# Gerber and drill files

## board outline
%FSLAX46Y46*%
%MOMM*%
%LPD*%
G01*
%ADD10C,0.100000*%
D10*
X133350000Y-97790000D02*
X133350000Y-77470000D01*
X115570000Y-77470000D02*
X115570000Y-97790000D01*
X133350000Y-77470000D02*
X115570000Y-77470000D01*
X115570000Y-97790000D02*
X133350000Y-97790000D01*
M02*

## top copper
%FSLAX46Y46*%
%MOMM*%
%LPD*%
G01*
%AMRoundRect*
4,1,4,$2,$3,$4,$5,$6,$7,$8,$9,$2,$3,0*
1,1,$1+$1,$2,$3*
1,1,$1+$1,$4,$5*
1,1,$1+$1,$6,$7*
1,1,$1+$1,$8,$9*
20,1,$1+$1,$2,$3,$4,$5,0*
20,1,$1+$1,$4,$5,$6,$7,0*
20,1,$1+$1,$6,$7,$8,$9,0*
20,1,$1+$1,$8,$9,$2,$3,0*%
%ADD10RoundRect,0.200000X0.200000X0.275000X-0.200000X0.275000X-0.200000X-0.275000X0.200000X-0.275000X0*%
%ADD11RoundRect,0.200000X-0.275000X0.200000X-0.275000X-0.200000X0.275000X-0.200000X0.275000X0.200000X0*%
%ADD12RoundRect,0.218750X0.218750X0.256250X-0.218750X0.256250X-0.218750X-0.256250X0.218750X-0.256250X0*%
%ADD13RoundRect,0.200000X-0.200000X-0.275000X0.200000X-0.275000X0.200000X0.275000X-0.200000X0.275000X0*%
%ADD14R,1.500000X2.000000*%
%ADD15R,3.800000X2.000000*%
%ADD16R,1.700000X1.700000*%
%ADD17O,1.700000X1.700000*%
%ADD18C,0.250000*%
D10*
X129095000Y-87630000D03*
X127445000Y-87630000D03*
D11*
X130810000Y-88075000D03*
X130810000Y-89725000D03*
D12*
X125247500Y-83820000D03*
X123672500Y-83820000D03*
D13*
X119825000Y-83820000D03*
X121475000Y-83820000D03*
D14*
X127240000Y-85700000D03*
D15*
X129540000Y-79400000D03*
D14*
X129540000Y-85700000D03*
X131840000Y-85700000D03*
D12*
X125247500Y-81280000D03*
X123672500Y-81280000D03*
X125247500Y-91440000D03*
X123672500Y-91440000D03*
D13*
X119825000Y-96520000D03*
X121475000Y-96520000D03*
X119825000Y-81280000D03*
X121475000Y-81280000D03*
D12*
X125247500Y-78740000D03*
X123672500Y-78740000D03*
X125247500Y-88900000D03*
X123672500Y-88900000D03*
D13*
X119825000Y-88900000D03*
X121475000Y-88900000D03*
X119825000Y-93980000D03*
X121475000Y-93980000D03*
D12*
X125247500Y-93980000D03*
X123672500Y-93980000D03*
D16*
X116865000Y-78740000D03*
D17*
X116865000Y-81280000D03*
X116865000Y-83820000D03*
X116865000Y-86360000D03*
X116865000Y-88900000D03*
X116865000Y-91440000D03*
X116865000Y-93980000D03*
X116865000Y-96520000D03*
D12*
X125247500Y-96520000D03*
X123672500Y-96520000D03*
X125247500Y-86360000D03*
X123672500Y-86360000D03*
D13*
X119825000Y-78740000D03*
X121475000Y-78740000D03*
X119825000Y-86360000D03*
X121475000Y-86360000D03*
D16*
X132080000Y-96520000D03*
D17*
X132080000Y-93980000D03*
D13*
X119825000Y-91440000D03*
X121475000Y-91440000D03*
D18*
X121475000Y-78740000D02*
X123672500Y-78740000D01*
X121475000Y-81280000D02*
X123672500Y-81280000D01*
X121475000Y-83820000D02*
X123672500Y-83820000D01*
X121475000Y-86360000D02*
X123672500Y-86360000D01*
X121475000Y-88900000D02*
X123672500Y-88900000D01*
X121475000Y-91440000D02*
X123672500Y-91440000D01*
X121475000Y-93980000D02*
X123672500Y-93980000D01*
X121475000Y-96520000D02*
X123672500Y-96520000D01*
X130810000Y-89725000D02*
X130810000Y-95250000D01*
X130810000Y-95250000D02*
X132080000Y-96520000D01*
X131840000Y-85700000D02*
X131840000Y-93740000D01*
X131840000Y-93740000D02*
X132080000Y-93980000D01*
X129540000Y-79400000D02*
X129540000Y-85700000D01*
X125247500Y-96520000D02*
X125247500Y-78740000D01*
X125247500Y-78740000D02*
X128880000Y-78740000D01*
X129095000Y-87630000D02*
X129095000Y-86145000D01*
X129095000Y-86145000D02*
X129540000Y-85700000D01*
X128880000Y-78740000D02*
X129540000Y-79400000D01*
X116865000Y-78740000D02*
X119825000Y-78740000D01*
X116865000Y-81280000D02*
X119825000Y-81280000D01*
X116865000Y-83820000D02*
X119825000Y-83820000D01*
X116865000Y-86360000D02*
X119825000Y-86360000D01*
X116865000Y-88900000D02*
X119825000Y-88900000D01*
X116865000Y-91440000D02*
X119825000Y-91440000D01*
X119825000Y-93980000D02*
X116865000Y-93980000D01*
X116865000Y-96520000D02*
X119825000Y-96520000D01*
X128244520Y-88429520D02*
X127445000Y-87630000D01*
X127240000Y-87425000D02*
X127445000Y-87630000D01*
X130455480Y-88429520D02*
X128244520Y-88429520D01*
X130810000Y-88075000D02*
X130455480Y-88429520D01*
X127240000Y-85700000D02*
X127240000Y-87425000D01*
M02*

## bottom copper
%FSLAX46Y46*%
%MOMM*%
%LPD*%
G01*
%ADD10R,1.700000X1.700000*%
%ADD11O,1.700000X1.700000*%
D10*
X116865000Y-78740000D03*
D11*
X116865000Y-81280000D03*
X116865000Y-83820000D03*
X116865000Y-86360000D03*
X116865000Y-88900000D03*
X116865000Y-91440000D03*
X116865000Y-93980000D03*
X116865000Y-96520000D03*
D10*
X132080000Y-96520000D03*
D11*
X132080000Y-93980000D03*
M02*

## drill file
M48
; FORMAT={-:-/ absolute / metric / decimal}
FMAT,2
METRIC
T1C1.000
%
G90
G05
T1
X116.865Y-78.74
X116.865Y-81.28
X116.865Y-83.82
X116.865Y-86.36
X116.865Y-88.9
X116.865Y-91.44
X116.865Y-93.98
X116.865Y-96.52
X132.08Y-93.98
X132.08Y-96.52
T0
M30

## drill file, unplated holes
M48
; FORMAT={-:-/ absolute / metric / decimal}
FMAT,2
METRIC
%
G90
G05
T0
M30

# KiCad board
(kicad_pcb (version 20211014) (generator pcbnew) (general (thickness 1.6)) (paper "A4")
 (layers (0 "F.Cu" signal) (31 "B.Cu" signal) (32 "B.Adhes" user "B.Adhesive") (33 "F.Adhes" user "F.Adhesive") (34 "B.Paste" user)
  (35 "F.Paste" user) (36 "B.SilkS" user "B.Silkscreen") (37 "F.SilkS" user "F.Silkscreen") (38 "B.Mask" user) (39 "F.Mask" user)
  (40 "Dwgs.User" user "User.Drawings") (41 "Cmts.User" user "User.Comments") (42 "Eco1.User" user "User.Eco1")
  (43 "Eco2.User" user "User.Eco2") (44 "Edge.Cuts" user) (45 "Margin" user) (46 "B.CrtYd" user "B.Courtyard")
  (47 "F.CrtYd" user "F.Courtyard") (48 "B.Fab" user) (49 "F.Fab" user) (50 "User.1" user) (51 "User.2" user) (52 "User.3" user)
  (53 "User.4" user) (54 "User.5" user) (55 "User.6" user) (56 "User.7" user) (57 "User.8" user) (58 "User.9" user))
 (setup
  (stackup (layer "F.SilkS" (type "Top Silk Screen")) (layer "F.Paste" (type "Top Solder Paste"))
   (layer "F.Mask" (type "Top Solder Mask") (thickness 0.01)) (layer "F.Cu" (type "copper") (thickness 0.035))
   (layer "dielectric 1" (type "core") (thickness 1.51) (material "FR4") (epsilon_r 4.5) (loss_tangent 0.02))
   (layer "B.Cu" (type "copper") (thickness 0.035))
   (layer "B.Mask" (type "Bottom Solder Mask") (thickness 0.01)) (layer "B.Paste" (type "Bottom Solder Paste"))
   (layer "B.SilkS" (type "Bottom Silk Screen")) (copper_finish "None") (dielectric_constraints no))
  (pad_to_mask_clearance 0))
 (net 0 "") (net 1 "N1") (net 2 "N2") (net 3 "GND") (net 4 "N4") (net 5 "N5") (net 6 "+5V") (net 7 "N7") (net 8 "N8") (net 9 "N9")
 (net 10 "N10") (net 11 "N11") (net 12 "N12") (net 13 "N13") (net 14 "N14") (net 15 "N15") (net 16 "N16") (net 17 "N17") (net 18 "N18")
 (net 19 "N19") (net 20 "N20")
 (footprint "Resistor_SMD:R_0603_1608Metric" (layer "F.Cu") (at 128.27 87.63 180)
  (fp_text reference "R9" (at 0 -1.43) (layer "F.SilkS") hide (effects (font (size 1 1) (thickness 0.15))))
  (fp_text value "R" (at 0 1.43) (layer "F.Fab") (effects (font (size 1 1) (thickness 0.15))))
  (pad "1" smd roundrect locked (at -0.825 0 180) (size 0.8 0.95) (layers "F.Cu" "F.Paste" "F.Mask") (roundrect_rratio 0.25) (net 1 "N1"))
  (pad "2" smd roundrect locked (at 0.825 0 180) (size 0.8 0.95) (layers "F.Cu" "F.Paste" "F.Mask") (roundrect_rratio 0.25) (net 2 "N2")))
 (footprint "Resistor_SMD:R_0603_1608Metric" (layer "F.Cu") (at 130.81 88.9 -90)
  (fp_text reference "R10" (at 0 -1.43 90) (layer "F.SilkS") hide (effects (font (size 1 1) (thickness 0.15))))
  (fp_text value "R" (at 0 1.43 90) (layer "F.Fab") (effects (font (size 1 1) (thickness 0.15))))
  (pad "1" smd roundrect locked (at -0.825 0 270) (size 0.8 0.95) (layers "F.Cu" "F.Paste" "F.Mask") (roundrect_rratio 0.25) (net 2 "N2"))
  (pad "2" smd roundrect locked (at 0.825 0 270) (size 0.8 0.95) (layers "F.Cu" "F.Paste" "F.Mask") (roundrect_rratio 0.25) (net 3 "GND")))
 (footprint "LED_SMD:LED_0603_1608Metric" (layer "F.Cu") (at 124.46 83.82 180)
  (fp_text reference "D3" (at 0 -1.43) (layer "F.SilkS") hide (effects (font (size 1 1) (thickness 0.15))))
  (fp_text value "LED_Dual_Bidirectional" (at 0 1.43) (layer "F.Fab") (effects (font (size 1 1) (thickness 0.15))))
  (pad "1" smd roundrect locked (at -0.7875 0 180) (size 0.875 0.95) (layers "F.Cu" "F.Paste" "F.Mask") (roundrect_rratio 0.25) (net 1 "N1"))
  (pad "2" smd roundrect locked (at 0.7875 0 180) (size 0.875 0.95) (layers "F.Cu" "F.Paste" "F.Mask") (roundrect_rratio 0.25) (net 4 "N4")))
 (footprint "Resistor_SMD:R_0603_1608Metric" (layer "F.Cu") (at 120.65 83.82)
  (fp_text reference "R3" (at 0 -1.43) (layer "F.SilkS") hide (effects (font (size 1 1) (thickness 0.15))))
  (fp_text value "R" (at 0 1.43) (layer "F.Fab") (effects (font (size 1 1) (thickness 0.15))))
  (pad "1" smd roundrect locked (at -0.825 0) (size 0.8 0.95) (layers "F.Cu" "F.Paste" "F.Mask") (roundrect_rratio 0.25) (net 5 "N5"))
  (pad "2" smd roundrect locked (at 0.825 0) (size 0.8 0.95) (layers "F.Cu" "F.Paste" "F.Mask") (roundrect_rratio 0.25) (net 4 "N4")))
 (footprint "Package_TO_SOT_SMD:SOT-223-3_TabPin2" (layer "F.Cu") (at 129.54 82.55 90)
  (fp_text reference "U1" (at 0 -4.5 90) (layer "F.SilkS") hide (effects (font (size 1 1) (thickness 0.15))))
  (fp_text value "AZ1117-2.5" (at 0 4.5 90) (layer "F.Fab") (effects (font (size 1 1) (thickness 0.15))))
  (pad "1" smd rect locked (at -3.15 -2.3 90) (size 2 1.5) (layers "F.Cu" "F.Paste" "F.Mask") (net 2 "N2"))
  (pad "2" smd rect locked (at 3.15 0 90) (size 2 3.8) (layers "F.Cu" "F.Paste" "F.Mask") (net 1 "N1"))
  (pad "2" smd rect locked (at -3.15 0 90) (size 2 1.5) (layers "F.Cu" "F.Paste" "F.Mask") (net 1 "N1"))
  (pad "3" smd rect locked (at -3.15 2.3 90) (size 2 1.5) (layers "F.Cu" "F.Paste" "F.Mask") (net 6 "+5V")))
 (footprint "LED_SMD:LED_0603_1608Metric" (layer "F.Cu") (at 124.46 81.28 180)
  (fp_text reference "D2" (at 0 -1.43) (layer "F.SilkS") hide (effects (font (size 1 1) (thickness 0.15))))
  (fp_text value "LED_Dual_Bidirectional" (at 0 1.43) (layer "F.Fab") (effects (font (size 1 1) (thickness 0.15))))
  (pad "1" smd roundrect locked (at -0.7875 0 180) (size 0.875 0.95) (layers "F.Cu" "F.Paste" "F.Mask") (roundrect_rratio 0.25) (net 1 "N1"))
  (pad "2" smd roundrect locked (at 0.7875 0 180) (size 0.875 0.95) (layers "F.Cu" "F.Paste" "F.Mask") (roundrect_rratio 0.25) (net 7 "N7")))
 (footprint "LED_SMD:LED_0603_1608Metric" (layer "F.Cu") (at 124.46 91.44 180)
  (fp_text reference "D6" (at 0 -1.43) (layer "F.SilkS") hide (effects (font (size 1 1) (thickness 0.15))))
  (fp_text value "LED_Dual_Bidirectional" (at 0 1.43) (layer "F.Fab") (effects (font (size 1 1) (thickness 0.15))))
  (pad "1" smd roundrect locked (at -0.7875 0 180) (size 0.875 0.95) (layers "F.Cu" "F.Paste" "F.Mask") (roundrect_rratio 0.25) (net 1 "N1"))
  (pad "2" smd roundrect locked (at 0.7875 0 180) (size 0.875 0.95) (layers "F.Cu" "F.Paste" "F.Mask") (roundrect_rratio 0.25) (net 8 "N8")))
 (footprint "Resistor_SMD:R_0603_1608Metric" (layer "F.Cu") (at 120.65 96.52)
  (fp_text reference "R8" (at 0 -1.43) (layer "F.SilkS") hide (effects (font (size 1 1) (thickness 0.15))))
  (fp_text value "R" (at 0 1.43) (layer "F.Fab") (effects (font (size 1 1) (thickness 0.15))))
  (pad "1" smd roundrect locked (at -0.825 0) (size 0.8 0.95) (layers "F.Cu" "F.Paste" "F.Mask") (roundrect_rratio 0.25) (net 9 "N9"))
  (pad "2" smd roundrect locked (at 0.825 0) (size 0.8 0.95) (layers "F.Cu" "F.Paste" "F.Mask") (roundrect_rratio 0.25) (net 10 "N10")))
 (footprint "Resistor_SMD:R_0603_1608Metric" (layer "F.Cu") (at 120.65 81.28)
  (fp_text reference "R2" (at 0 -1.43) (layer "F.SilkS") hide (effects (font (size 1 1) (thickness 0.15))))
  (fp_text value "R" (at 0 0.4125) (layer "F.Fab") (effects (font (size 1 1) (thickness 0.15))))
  (pad "1" smd roundrect locked (at -0.825 0) (size 0.8 0.95) (layers "F.Cu" "F.Paste" "F.Mask") (roundrect_rratio 0.25) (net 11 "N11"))
  (pad "2" smd roundrect locked (at 0.825 0) (size 0.8 0.95) (layers "F.Cu" "F.Paste" "F.Mask") (roundrect_rratio 0.25) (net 7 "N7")))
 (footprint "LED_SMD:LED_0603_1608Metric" (layer "F.Cu") (at 124.46 78.74 180)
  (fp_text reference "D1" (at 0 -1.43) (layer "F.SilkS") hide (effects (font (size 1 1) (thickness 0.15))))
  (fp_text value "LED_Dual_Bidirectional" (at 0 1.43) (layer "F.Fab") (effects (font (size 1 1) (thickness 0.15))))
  (pad "1" smd roundrect locked (at -0.7875 0 180) (size 0.875 0.95) (layers "F.Cu" "F.Paste" "F.Mask") (roundrect_rratio 0.25) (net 1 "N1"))
  (pad "2" smd roundrect locked (at 0.7875 0 180) (size 0.875 0.95) (layers "F.Cu" "F.Paste" "F.Mask") (roundrect_rratio 0.25)
   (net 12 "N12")))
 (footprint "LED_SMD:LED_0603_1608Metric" (layer "F.Cu") (at 124.46 88.9 180)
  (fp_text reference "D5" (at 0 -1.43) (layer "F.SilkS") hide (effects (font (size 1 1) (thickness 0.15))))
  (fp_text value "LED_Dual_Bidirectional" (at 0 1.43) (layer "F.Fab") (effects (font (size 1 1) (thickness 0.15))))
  (pad "1" smd roundrect locked (at -0.7875 0 180) (size 0.875 0.95) (layers "F.Cu" "F.Paste" "F.Mask") (roundrect_rratio 0.25) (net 1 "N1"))
  (pad "2" smd roundrect locked (at 0.7875 0 180) (size 0.875 0.95) (layers "F.Cu" "F.Paste" "F.Mask") (roundrect_rratio 0.25)
   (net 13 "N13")))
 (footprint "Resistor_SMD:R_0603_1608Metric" (layer "F.Cu") (at 120.65 88.9)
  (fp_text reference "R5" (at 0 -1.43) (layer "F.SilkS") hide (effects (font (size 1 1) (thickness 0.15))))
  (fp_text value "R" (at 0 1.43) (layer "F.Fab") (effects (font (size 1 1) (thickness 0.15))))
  (pad "1" smd roundrect locked (at -0.825 0) (size 0.8 0.95) (layers "F.Cu" "F.Paste" "F.Mask") (roundrect_rratio 0.25) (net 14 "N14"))
  (pad "2" smd roundrect locked (at 0.825 0) (size 0.8 0.95) (layers "F.Cu" "F.Paste" "F.Mask") (roundrect_rratio 0.25) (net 13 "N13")))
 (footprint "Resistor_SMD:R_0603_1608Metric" (layer "F.Cu") (at 120.65 93.98)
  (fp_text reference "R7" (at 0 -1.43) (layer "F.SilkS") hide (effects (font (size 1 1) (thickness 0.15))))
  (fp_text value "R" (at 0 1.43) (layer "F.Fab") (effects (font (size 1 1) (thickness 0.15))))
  (pad "1" smd roundrect locked (at -0.825 0) (size 0.8 0.95) (layers "F.Cu" "F.Paste" "F.Mask") (roundrect_rratio 0.25) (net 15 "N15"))
  (pad "2" smd roundrect locked (at 0.825 0) (size 0.8 0.95) (layers "F.Cu" "F.Paste" "F.Mask") (roundrect_rratio 0.25) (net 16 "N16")))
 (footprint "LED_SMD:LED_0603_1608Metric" (layer "F.Cu") (at 124.46 93.98 180)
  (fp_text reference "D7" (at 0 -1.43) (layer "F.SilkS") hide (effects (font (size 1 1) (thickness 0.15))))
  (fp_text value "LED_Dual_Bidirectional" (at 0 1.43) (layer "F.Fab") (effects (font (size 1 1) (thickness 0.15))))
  (pad "1" smd roundrect locked (at -0.7875 0 180) (size 0.875 0.95) (layers "F.Cu" "F.Paste" "F.Mask") (roundrect_rratio 0.25) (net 1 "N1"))
  (pad "2" smd roundrect locked (at 0.7875 0 180) (size 0.875 0.95) (layers "F.Cu" "F.Paste" "F.Mask") (roundrect_rratio 0.25)
   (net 16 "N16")))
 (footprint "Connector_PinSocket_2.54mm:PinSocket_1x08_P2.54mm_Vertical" (layer "F.Cu") (at 116.865 78.74)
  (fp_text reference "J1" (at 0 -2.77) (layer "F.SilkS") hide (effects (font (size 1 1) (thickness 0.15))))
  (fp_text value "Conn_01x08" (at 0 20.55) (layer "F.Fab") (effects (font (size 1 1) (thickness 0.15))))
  (pad "1" thru_hole rect locked (at 0 0) (size 1.7 1.7) (drill 1) (layers *.Cu *.Mask) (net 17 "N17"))
  (pad "2" thru_hole oval locked (at 0 2.54) (size 1.7 1.7) (drill 1) (layers *.Cu *.Mask) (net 11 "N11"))
  (pad "3" thru_hole oval locked (at 0 5.08) (size 1.7 1.7) (drill 1) (layers *.Cu *.Mask) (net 5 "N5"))
  (pad "4" thru_hole oval locked (at 0 7.62) (size 1.7 1.7) (drill 1) (layers *.Cu *.Mask) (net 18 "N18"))
  (pad "5" thru_hole oval locked (at 0 10.16) (size 1.7 1.7) (drill 1) (layers *.Cu *.Mask) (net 14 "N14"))
  (pad "6" thru_hole oval locked (at 0 12.7) (size 1.7 1.7) (drill 1) (layers *.Cu *.Mask) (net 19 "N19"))
  (pad "7" thru_hole oval locked (at 0 15.24) (size 1.7 1.7) (drill 1) (layers *.Cu *.Mask) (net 15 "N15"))
  (pad "8" thru_hole oval locked (at 0 17.78) (size 1.7 1.7) (drill 1) (layers *.Cu *.Mask) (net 9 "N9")))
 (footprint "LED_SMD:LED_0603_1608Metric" (layer "F.Cu") (at 124.46 96.52 180)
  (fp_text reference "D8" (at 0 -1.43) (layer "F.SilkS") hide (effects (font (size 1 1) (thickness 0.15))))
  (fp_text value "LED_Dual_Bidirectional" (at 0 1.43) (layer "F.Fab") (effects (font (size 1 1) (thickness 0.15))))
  (pad "1" smd roundrect locked (at -0.7875 0 180) (size 0.875 0.95) (layers "F.Cu" "F.Paste" "F.Mask") (roundrect_rratio 0.25) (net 1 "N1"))
  (pad "2" smd roundrect locked (at 0.7875 0 180) (size 0.875 0.95) (layers "F.Cu" "F.Paste" "F.Mask") (roundrect_rratio 0.25)
   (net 10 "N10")))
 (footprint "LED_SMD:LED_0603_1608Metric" (layer "F.Cu") (at 124.46 86.36 180)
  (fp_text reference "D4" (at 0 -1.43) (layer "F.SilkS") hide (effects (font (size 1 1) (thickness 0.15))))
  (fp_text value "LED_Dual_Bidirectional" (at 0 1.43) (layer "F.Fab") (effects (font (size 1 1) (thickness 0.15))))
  (pad "1" smd roundrect locked (at -0.7875 0 180) (size 0.875 0.95) (layers "F.Cu" "F.Paste" "F.Mask") (roundrect_rratio 0.25) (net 1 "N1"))
  (pad "2" smd roundrect locked (at 0.7875 0 180) (size 0.875 0.95) (layers "F.Cu" "F.Paste" "F.Mask") (roundrect_rratio 0.25)
   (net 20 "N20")))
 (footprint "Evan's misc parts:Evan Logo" (layer "F.Cu") (at 128.27 90.932)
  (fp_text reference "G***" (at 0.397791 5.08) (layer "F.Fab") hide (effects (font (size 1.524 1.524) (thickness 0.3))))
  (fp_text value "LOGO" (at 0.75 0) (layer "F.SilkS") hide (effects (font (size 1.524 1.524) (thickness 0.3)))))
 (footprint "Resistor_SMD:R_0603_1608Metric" (layer "F.Cu") (at 120.65 78.74)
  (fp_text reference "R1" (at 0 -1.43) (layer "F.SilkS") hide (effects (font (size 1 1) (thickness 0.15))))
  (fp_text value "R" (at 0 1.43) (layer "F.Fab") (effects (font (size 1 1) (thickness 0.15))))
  (pad "1" smd roundrect locked (at -0.825 0) (size 0.8 0.95) (layers "F.Cu" "F.Paste" "F.Mask") (roundrect_rratio 0.25) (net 17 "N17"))
  (pad "2" smd roundrect locked (at 0.825 0) (size 0.8 0.95) (layers "F.Cu" "F.Paste" "F.Mask") (roundrect_rratio 0.25) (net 12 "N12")))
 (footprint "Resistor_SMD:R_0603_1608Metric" (layer "F.Cu") (at 120.65 86.36)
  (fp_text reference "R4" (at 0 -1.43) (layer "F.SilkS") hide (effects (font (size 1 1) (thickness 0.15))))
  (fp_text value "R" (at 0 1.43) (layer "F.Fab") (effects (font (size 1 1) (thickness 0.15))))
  (pad "1" smd roundrect locked (at -0.825 0) (size 0.8 0.95) (layers "F.Cu" "F.Paste" "F.Mask") (roundrect_rratio 0.25) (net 18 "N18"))
  (pad "2" smd roundrect locked (at 0.825 0) (size 0.8 0.95) (layers "F.Cu" "F.Paste" "F.Mask") (roundrect_rratio 0.25) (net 20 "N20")))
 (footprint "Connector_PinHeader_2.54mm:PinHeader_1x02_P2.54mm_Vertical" (layer "F.Cu") (at 132.08 96.52 180)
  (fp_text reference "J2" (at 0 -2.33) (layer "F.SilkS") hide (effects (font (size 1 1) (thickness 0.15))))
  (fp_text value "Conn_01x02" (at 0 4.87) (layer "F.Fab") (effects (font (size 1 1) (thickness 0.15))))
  (pad "1" thru_hole rect locked (at 0 0 180) (size 1.7 1.7) (drill 1) (layers *.Cu *.Mask) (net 3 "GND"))
  (pad "2" thru_hole oval locked (at 0 2.54 180) (size 1.7 1.7) (drill 1) (layers *.Cu *.Mask) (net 6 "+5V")))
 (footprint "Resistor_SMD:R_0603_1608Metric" (layer "F.Cu") (at 120.65 91.44)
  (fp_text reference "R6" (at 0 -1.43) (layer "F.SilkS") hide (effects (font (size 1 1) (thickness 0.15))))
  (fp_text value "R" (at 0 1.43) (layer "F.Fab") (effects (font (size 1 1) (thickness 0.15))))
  (pad "1" smd roundrect locked (at -0.825 0) (size 0.8 0.95) (layers "F.Cu" "F.Paste" "F.Mask") (roundrect_rratio 0.25) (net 19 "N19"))
  (pad "2" smd roundrect locked (at 0.825 0) (size 0.8 0.95) (layers "F.Cu" "F.Paste" "F.Mask") (roundrect_rratio 0.25) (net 8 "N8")))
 (gr_line (start 133.35 97.79) (end 133.35 77.47) (layer "Edge.Cuts") (width 0.1))
 (gr_line (start 115.57 77.47) (end 115.57 97.79) (layer "Edge.Cuts") (width 0.1))
 (gr_line (start 133.35 77.47) (end 115.57 77.47) (layer "Edge.Cuts") (width 0.1))
 (gr_line (start 115.57 97.79) (end 133.35 97.79) (layer "Edge.Cuts") (width 0.1))
 (segment (start 121.475 78.74) (end 123.6725 78.74) (width 0.25) (layer "F.Cu") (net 12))
 (segment (start 121.475 81.28) (end 123.6725 81.28) (width 0.25) (layer "F.Cu") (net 7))
 (segment (start 121.475 83.82) (end 123.6725 83.82) (width 0.25) (layer "F.Cu") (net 4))
 (segment (start 121.475 86.36) (end 123.6725 86.36) (width 0.25) (layer "F.Cu") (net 20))
 (segment (start 121.475 88.9) (end 123.6725 88.9) (width 0.25) (layer "F.Cu") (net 13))
 (segment (start 121.475 91.44) (end 123.6725 91.44) (width 0.25) (layer "F.Cu") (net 8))
 (segment (start 121.475 93.98) (end 123.6725 93.98) (width 0.25) (layer "F.Cu") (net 16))
 (segment (start 121.475 96.52) (end 123.6725 96.52) (width 0.25) (layer "F.Cu") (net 10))
 (segment (start 130.81 89.725) (end 130.81 95.25) (width 0.25) (layer "F.Cu") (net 3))
 (segment (start 130.81 95.25) (end 132.08 96.52) (width 0.25) (layer "F.Cu") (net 3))
 (segment (start 131.84 85.7) (end 131.84 93.74) (width 0.25) (layer "F.Cu") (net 6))
 (segment (start 131.84 93.74) (end 132.08 93.98) (width 0.25) (layer "F.Cu") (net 6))
 (segment (start 129.54 79.4) (end 129.54 85.7) (width 0.25) (layer "F.Cu") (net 1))
 (segment (start 125.2475 96.52) (end 125.2475 78.74) (width 0.25) (layer "F.Cu") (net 1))
 (segment (start 125.2475 78.74) (end 128.88 78.74) (width 0.25) (layer "F.Cu") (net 1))
 (segment (start 129.095 87.63) (end 129.095 86.145) (width 0.25) (layer "F.Cu") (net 1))
 (segment (start 129.095 86.145) (end 129.54 85.7) (width 0.25) (layer "F.Cu") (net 1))
 (segment (start 128.88 78.74) (end 129.54 79.4) (width 0.25) (layer "F.Cu") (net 1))
 (segment (start 116.865 78.74) (end 119.825 78.74) (width 0.25) (layer "F.Cu") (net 17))
 (segment (start 116.865 81.28) (end 119.825 81.28) (width 0.25) (layer "F.Cu") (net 11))
 (segment (start 116.865 83.82) (end 119.825 83.82) (width 0.25) (layer "F.Cu") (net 5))
 (segment (start 116.865 86.36) (end 119.825 86.36) (width 0.25) (layer "F.Cu") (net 18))
 (segment (start 116.865 88.9) (end 119.825 88.9) (width 0.25) (layer "F.Cu") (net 14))
 (segment (start 116.865 91.44) (end 119.825 91.44) (width 0.25) (layer "F.Cu") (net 19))
 (segment (start 119.825 93.98) (end 116.865 93.98) (width 0.25) (layer "F.Cu") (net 15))
 (segment (start 116.865 96.52) (end 119.825 96.52) (width 0.25) (layer "F.Cu") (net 9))
 (segment (start 128.24452 88.42952) (end 127.445 87.63) (width 0.25) (layer "F.Cu") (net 2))
 (segment (start 127.24 87.425) (end 127.445 87.63) (width 0.25) (layer "F.Cu") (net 2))
 (segment (start 130.45548 88.42952) (end 128.24452 88.42952) (width 0.25) (layer "F.Cu") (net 2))
 (segment (start 130.81 88.075) (end 130.45548 88.42952) (width 0.25) (layer "F.Cu") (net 2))
 (segment (start 127.24 85.7) (end 127.24 87.425) (width 0.25) (layer "F.Cu") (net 2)))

